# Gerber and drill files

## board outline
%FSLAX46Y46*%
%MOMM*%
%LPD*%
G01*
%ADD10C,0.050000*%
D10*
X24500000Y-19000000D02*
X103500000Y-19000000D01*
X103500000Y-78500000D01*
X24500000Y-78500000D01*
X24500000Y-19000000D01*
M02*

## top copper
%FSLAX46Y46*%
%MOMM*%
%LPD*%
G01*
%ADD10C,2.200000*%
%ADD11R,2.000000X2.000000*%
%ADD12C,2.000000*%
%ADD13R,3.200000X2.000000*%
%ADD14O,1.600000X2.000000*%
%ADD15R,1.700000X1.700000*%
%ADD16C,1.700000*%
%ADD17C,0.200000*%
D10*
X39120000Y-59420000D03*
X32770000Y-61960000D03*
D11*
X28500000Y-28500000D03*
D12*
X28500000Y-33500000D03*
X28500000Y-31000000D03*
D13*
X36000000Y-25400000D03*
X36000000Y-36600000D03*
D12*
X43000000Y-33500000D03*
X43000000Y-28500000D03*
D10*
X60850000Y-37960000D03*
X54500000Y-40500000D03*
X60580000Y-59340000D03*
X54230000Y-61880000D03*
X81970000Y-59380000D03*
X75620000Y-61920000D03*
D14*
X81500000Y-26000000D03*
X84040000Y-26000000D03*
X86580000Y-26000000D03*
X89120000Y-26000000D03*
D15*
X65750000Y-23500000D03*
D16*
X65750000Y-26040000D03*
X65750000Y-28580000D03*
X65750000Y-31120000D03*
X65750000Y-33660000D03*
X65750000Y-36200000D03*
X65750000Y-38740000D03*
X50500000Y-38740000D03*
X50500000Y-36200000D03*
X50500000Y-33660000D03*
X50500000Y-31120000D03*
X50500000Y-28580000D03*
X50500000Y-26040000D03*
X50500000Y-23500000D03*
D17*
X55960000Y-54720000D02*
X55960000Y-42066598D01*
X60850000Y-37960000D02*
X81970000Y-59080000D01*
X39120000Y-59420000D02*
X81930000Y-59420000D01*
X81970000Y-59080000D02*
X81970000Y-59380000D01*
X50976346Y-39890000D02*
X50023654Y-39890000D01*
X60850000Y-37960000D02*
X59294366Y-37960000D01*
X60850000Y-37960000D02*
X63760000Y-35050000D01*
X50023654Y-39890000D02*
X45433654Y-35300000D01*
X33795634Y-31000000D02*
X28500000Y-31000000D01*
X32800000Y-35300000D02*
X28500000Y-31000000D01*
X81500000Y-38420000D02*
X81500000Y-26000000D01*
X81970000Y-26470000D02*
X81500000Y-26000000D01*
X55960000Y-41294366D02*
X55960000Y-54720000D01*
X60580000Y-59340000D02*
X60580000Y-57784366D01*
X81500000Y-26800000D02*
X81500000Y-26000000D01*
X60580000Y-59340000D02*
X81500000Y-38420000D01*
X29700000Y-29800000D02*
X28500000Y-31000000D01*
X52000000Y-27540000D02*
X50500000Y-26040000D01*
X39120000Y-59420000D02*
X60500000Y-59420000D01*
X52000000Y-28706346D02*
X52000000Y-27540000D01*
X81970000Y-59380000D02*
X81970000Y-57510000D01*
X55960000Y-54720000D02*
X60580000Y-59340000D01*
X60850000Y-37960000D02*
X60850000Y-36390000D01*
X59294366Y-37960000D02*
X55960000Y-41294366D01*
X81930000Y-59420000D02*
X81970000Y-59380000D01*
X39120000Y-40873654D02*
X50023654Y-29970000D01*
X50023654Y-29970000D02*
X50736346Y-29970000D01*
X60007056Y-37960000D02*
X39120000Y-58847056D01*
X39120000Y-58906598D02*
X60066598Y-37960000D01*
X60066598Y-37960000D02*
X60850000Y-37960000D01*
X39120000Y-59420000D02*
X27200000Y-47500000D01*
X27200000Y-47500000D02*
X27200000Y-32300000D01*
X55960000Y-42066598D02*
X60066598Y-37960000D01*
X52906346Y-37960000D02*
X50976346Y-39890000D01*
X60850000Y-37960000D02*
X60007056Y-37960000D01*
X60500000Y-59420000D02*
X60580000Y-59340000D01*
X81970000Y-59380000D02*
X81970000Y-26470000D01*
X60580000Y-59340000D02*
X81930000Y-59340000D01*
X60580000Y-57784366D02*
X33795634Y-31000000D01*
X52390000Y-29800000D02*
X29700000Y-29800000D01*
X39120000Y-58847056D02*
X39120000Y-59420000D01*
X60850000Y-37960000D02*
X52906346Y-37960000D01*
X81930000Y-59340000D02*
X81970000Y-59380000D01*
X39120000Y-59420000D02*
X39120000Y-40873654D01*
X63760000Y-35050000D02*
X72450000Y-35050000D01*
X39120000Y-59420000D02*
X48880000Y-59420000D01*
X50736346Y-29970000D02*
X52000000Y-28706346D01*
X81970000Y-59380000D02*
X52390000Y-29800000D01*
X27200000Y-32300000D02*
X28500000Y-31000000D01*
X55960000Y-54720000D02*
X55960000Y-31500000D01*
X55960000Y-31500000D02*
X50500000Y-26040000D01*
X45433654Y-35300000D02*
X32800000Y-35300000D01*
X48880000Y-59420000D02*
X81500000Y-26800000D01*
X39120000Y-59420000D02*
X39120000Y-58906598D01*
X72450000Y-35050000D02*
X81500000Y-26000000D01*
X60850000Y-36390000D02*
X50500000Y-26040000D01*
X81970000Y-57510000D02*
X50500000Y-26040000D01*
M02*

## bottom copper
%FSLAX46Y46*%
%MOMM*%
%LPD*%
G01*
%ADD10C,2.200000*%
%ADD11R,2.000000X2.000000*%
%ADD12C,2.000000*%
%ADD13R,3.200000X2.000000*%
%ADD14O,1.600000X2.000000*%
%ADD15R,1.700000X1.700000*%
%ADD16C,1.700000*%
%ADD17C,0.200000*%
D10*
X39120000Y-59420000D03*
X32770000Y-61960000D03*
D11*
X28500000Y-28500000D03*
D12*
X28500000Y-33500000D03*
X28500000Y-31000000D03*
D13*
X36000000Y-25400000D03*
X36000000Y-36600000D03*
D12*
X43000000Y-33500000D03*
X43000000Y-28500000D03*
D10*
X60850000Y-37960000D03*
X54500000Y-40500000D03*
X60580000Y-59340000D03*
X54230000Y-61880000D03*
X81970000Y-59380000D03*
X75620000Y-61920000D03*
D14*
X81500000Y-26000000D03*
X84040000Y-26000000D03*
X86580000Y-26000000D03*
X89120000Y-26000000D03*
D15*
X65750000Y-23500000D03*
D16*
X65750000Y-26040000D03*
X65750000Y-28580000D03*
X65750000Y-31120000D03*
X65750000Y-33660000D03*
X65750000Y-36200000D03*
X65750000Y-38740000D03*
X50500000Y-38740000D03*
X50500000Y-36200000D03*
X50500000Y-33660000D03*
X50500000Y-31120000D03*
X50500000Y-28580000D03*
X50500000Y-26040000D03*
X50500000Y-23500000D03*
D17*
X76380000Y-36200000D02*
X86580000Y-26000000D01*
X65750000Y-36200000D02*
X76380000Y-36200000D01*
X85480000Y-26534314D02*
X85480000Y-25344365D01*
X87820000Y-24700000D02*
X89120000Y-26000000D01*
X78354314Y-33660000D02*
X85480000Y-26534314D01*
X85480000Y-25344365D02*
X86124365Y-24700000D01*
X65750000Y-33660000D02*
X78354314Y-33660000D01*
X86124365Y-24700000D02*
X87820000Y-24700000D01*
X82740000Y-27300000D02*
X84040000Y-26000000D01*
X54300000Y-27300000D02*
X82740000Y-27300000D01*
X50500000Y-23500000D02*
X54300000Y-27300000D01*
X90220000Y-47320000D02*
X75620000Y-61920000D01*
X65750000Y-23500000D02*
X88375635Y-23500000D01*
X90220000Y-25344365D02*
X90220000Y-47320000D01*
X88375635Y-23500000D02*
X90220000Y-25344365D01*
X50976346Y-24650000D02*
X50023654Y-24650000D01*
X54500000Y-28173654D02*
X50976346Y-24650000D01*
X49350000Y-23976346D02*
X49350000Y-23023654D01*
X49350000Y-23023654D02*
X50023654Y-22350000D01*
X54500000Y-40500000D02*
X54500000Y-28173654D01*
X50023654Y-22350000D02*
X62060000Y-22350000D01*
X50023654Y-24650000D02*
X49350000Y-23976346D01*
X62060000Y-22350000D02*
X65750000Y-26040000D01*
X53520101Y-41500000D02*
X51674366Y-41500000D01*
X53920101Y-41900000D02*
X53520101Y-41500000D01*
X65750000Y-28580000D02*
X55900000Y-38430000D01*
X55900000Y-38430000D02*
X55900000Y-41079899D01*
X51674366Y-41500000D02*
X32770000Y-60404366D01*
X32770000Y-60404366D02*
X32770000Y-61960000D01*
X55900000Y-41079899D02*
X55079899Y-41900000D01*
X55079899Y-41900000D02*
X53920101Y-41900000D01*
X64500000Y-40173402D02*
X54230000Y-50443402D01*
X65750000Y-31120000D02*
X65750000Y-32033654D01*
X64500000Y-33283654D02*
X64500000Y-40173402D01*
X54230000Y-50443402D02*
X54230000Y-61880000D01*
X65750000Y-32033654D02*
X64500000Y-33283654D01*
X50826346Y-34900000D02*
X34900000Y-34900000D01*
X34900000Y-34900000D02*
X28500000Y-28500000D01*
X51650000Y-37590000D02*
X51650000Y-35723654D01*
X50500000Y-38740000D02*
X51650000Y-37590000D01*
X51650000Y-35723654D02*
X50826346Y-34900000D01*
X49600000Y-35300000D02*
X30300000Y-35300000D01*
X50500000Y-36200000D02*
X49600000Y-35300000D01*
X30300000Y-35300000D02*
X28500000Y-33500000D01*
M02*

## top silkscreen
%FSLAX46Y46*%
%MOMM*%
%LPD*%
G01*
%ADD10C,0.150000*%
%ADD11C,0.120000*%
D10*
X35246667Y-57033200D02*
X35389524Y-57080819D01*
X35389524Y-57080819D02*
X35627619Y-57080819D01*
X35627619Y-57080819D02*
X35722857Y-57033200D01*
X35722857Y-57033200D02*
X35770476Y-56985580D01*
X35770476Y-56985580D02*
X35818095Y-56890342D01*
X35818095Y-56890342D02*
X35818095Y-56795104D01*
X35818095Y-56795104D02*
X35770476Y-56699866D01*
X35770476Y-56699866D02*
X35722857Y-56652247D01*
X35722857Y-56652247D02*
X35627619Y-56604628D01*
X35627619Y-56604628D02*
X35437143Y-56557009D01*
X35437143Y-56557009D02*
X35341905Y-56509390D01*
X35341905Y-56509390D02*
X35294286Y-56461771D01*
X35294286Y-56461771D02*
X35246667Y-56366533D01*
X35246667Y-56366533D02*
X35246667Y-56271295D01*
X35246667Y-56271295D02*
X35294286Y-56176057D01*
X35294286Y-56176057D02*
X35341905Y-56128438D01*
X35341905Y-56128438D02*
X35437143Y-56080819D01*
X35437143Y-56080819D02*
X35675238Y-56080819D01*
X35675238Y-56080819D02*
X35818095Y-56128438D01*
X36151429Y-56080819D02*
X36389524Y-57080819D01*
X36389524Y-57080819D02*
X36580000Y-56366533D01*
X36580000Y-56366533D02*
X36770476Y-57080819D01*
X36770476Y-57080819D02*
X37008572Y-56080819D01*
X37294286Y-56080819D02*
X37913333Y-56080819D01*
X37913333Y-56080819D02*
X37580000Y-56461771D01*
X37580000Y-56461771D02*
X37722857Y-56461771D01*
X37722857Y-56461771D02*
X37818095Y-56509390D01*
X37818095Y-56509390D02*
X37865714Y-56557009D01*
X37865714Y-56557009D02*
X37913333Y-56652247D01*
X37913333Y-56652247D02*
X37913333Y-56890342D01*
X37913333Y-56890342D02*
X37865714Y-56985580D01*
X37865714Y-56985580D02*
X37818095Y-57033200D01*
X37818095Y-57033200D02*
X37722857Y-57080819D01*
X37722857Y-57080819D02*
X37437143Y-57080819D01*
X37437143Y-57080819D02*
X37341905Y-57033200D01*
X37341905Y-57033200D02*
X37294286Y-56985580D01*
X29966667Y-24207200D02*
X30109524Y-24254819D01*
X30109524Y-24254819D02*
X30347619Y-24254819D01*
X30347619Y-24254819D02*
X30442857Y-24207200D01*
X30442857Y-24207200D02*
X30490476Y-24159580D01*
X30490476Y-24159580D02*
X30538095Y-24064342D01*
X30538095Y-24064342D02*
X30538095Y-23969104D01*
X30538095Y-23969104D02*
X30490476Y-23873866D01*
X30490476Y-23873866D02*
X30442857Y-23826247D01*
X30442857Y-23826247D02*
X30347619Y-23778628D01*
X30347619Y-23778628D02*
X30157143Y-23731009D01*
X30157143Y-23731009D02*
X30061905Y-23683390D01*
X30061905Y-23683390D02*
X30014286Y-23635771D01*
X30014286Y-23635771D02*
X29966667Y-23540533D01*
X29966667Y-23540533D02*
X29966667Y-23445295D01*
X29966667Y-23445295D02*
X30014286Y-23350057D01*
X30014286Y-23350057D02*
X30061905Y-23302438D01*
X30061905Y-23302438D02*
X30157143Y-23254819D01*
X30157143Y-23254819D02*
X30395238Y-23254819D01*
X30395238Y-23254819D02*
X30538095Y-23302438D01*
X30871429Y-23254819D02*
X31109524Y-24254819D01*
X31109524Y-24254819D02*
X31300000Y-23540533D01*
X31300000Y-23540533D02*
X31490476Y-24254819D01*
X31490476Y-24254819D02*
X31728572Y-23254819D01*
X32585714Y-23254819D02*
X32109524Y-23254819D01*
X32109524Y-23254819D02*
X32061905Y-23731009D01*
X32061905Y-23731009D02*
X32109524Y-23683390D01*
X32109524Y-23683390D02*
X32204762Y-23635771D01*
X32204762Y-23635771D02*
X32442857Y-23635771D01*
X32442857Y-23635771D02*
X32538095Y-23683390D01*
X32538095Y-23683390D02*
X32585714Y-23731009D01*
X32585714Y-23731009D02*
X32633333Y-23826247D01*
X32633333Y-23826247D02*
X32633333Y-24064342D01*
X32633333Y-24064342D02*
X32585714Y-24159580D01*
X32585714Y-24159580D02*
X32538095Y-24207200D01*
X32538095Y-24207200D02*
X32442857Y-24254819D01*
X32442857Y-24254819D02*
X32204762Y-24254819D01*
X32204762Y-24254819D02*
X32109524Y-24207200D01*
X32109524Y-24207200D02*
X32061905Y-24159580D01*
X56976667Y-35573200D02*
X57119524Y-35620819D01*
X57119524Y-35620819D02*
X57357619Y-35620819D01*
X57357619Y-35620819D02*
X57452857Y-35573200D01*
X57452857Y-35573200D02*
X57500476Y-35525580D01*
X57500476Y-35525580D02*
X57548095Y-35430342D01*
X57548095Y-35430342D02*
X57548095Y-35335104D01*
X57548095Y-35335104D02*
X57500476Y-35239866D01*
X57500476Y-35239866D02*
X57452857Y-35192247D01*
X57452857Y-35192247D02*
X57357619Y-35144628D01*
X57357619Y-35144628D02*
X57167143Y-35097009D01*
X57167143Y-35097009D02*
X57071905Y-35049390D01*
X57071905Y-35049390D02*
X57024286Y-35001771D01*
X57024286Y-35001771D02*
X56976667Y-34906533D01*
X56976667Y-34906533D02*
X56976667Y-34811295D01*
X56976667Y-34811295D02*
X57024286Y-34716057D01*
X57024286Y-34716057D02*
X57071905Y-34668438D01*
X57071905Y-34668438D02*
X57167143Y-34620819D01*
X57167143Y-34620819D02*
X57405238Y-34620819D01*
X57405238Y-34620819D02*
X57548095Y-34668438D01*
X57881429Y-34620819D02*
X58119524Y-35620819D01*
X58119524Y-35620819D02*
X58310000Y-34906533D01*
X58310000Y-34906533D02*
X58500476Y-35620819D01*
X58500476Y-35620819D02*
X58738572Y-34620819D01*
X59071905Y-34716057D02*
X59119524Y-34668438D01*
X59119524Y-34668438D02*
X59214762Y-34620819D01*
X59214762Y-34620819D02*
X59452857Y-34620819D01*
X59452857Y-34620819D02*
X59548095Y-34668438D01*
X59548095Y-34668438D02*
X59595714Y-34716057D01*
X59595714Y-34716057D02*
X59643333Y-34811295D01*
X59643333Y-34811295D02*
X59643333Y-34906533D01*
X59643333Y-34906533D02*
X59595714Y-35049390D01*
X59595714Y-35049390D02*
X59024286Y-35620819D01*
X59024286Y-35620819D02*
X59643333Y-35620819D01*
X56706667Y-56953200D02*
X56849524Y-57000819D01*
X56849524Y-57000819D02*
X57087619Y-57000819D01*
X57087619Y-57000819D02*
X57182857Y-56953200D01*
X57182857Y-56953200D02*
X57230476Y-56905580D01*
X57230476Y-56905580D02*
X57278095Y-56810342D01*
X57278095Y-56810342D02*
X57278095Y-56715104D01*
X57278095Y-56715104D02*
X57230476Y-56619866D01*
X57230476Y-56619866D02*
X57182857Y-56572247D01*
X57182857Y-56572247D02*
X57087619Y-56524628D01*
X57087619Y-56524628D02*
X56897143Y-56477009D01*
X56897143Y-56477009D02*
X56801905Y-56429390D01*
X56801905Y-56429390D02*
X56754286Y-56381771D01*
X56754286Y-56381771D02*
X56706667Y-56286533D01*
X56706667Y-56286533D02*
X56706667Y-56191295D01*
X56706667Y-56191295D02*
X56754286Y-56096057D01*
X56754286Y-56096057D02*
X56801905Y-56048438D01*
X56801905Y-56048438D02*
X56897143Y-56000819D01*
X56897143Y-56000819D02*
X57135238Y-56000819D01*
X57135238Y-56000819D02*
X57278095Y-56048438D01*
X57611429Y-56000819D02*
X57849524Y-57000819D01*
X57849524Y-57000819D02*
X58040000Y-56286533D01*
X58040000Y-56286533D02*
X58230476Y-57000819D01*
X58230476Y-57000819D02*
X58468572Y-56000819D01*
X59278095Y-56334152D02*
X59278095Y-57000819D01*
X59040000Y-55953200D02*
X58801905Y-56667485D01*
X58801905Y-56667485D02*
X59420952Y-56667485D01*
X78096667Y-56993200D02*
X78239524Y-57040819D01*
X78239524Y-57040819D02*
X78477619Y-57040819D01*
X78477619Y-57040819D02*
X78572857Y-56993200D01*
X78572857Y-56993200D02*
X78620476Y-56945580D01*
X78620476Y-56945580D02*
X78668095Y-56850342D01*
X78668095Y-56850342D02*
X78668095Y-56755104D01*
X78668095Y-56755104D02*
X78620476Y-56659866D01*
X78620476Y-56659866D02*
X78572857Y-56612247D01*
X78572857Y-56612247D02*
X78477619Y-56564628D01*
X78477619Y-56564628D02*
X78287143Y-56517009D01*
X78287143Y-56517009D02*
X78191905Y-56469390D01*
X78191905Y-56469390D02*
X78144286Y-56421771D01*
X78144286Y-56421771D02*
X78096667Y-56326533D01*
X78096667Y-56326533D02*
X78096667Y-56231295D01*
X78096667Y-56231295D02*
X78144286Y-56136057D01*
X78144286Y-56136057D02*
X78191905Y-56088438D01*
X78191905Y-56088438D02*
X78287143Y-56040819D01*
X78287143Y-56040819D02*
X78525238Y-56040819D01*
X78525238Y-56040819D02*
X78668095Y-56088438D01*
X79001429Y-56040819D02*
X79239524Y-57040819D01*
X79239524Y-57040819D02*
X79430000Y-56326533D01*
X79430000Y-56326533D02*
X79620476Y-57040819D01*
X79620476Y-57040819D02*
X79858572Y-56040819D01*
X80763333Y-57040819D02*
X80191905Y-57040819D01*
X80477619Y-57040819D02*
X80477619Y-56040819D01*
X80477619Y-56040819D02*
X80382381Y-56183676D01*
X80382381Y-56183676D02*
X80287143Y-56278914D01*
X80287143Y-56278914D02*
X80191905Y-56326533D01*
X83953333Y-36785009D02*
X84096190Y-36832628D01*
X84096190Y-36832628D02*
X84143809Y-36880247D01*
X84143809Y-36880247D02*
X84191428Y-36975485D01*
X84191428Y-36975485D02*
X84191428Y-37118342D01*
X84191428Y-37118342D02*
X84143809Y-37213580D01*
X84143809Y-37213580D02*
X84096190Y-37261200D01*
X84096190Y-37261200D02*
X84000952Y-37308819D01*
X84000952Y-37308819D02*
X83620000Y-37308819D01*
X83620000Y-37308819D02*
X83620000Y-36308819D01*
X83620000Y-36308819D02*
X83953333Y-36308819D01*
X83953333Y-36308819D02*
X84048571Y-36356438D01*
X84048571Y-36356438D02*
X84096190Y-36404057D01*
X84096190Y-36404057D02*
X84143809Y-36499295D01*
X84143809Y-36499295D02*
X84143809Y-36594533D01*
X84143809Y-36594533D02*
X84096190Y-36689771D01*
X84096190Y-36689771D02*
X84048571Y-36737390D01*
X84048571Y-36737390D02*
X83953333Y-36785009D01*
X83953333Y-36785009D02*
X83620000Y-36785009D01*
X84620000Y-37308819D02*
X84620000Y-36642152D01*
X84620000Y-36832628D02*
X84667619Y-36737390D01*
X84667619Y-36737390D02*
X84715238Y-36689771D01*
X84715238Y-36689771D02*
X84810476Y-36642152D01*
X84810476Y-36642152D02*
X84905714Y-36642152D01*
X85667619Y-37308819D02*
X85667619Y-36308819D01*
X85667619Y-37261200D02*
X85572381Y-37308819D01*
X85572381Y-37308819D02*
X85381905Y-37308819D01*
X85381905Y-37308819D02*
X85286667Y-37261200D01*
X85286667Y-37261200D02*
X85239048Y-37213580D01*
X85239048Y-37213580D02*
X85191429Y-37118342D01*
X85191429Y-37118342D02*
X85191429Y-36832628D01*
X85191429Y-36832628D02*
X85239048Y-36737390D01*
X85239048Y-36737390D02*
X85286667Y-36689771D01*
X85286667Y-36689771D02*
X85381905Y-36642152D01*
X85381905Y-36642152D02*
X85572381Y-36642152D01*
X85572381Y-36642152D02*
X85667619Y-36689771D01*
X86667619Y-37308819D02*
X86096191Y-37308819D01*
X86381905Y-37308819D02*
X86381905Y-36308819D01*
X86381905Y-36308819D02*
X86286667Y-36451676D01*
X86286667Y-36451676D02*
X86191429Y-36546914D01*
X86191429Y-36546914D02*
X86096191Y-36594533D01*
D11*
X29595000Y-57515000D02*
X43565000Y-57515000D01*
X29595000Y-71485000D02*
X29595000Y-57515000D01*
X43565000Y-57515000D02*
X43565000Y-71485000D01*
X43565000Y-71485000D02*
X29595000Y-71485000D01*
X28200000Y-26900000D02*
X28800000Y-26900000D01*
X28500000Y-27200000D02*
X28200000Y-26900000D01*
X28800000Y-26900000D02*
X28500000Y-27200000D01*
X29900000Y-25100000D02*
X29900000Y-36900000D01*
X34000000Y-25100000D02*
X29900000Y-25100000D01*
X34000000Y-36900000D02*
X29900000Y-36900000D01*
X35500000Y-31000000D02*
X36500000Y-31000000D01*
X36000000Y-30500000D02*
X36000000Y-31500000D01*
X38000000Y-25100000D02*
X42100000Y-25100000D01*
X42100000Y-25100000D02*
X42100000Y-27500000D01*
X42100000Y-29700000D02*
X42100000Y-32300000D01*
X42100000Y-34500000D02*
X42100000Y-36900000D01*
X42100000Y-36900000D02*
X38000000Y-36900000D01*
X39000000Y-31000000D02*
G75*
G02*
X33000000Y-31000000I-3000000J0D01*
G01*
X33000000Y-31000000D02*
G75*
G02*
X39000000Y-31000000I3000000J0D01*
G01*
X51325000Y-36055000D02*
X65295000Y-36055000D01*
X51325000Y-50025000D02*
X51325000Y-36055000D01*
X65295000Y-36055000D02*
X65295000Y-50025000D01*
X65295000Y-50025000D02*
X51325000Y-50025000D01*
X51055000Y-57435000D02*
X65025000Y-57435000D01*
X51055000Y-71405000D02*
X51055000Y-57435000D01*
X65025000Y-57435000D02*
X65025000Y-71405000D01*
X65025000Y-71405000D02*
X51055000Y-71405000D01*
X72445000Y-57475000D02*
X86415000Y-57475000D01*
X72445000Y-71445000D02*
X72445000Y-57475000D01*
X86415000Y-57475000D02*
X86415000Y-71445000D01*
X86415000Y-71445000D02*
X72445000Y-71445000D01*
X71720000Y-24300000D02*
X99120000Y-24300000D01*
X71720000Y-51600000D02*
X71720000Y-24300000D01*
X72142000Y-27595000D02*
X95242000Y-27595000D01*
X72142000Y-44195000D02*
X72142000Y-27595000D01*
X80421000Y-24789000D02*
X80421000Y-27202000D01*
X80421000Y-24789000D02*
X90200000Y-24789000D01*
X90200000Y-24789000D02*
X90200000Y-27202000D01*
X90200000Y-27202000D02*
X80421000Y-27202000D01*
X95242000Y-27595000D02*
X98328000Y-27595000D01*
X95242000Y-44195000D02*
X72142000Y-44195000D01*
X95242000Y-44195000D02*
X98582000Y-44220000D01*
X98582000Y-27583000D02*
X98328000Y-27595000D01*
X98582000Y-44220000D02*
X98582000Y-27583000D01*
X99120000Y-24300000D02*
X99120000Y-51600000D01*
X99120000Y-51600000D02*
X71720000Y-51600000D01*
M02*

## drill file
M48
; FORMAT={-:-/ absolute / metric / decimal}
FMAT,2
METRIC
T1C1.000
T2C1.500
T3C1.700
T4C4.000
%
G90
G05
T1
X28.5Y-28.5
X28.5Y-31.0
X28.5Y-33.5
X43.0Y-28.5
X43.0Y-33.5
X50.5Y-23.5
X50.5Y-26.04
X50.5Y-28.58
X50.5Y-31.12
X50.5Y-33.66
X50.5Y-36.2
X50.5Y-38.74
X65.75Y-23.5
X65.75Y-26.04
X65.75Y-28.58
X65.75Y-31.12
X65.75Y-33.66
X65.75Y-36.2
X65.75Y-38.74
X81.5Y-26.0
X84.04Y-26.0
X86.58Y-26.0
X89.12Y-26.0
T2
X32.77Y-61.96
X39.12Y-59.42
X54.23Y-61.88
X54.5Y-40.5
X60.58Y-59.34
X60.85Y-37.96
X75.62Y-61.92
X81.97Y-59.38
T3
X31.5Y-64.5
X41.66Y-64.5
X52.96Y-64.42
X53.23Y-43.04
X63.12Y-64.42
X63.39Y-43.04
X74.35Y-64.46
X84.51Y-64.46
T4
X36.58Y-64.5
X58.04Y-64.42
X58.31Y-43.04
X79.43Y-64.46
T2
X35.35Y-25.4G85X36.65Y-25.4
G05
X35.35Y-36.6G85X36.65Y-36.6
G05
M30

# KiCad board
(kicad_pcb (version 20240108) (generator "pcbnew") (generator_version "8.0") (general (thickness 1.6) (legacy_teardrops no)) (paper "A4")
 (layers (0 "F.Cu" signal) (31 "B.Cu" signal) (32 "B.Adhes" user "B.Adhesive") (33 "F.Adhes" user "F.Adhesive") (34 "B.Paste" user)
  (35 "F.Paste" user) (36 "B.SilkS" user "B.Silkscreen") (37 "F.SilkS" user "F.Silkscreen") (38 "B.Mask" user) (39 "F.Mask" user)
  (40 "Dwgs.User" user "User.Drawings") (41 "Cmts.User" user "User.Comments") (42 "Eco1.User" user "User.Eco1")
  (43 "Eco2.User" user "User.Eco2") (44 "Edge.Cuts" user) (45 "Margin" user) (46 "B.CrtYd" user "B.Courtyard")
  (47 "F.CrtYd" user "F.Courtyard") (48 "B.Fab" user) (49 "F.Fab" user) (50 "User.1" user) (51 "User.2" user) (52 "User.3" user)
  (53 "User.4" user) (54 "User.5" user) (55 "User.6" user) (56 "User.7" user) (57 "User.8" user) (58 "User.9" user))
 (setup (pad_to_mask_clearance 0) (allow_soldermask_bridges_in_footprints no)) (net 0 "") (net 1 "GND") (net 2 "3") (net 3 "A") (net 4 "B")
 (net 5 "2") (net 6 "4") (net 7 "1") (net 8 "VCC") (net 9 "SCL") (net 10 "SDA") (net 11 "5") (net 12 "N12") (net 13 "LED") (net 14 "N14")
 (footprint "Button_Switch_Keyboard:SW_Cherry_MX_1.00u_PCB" (layer "F.Cu") (at 39.12 59.42)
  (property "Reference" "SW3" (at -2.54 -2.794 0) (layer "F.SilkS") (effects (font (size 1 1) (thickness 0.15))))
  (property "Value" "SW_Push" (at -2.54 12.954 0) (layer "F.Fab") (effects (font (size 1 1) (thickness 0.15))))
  (fp_line (start -9.525 -1.905) (end 4.445 -1.905) (stroke (width 0.12) (type solid)) (layer "F.SilkS"))
  (fp_line (start -9.525 12.065) (end -9.525 -1.905) (stroke (width 0.12) (type solid)) (layer "F.SilkS"))
  (fp_line (start 4.445 -1.905) (end 4.445 12.065) (stroke (width 0.12) (type solid)) (layer "F.SilkS"))
  (fp_line (start 4.445 12.065) (end -9.525 12.065) (stroke (width 0.12) (type solid)) (layer "F.SilkS"))
  (pad "" np_thru_hole circle (at -7.62 5.08) (size 1.7 1.7) (drill 1.7) (layers "*.Cu" "*.Mask"))
  (pad "" np_thru_hole circle (at -2.54 5.08) (size 4 4) (drill 4) (layers "*.Cu" "*.Mask"))
  (pad "" np_thru_hole circle (at 2.54 5.08) (size 1.7 1.7) (drill 1.7) (layers "*.Cu" "*.Mask"))
  (pad "1" thru_hole circle (at 0 0) (size 2.2 2.2) (drill 1.5) (layers "*.Cu" "*.Mask") (remove_unused_layers no) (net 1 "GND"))
  (pad "2" thru_hole circle (at -6.35 2.54) (size 2.2 2.2) (drill 1.5) (layers "*.Cu" "*.Mask") (remove_unused_layers no) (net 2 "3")))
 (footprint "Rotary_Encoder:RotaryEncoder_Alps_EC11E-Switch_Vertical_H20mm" (layer "F.Cu") (at 28.5 28.5)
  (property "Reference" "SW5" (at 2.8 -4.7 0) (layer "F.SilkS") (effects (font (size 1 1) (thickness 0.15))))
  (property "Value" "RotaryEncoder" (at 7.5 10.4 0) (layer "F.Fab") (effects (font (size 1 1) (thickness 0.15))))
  (fp_line (start -0.3 -1.6) (end 0.3 -1.6) (stroke (width 0.12) (type solid)) (layer "F.SilkS"))
  (fp_line (start 0 -1.3) (end -0.3 -1.6) (stroke (width 0.12) (type solid)) (layer "F.SilkS"))
  (fp_line (start 0.3 -1.6) (end 0 -1.3) (stroke (width 0.12) (type solid)) (layer "F.SilkS"))
  (fp_line (start 1.4 -3.4) (end 1.4 8.4) (stroke (width 0.12) (type solid)) (layer "F.SilkS"))
  (fp_line (start 5.5 -3.4) (end 1.4 -3.4) (stroke (width 0.12) (type solid)) (layer "F.SilkS"))
  (fp_line (start 5.5 8.4) (end 1.4 8.4) (stroke (width 0.12) (type solid)) (layer "F.SilkS"))
  (fp_line (start 7 2.5) (end 8 2.5) (stroke (width 0.12) (type solid)) (layer "F.SilkS"))
  (fp_line (start 7.5 2) (end 7.5 3) (stroke (width 0.12) (type solid)) (layer "F.SilkS"))
  (fp_line (start 9.5 -3.4) (end 13.6 -3.4) (stroke (width 0.12) (type solid)) (layer "F.SilkS"))
  (fp_line (start 13.6 -3.4) (end 13.6 -1) (stroke (width 0.12) (type solid)) (layer "F.SilkS"))
  (fp_line (start 13.6 1.2) (end 13.6 3.8) (stroke (width 0.12) (type solid)) (layer "F.SilkS"))
  (fp_line (start 13.6 6) (end 13.6 8.4) (stroke (width 0.12) (type solid)) (layer "F.SilkS"))
  (fp_line (start 13.6 8.4) (end 9.5 8.4) (stroke (width 0.12) (type solid)) (layer "F.SilkS"))
  (fp_circle (center 7.5 2.5) (end 10.5 2.5) (stroke (width 0.12) (type solid)) (fill none) (layer "F.SilkS"))
  (pad "A" thru_hole rect (at 0 0) (size 2 2) (drill 1) (layers "*.Cu" "*.Mask") (remove_unused_layers no) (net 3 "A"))
  (pad "B" thru_hole circle (at 0 5) (size 2 2) (drill 1) (layers "*.Cu" "*.Mask") (remove_unused_layers no) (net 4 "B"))
  (pad "C" thru_hole circle (at 0 2.5) (size 2 2) (drill 1) (layers "*.Cu" "*.Mask") (remove_unused_layers no) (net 1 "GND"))
  (pad "MP" thru_hole rect (at 7.5 -3.1) (size 3.2 2) (drill oval 2.8 1.5) (layers "*.Cu" "*.Mask") (remove_unused_layers no))
  (pad "MP" thru_hole rect (at 7.5 8.1) (size 3.2 2) (drill oval 2.8 1.5) (layers "*.Cu" "*.Mask") (remove_unused_layers no))
  (pad "S1" thru_hole circle (at 14.5 5) (size 2 2) (drill 1) (layers "*.Cu" "*.Mask") (remove_unused_layers no))
  (pad "S2" thru_hole circle (at 14.5 0) (size 2 2) (drill 1) (layers "*.Cu" "*.Mask") (remove_unused_layers no)))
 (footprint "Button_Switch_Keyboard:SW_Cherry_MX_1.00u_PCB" (layer "F.Cu") (at 60.85 37.96)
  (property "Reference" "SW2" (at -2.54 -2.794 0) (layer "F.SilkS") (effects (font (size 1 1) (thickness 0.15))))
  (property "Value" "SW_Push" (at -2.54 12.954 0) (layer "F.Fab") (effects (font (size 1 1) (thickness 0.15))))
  (fp_line (start -9.525 -1.905) (end 4.445 -1.905) (stroke (width 0.12) (type solid)) (layer "F.SilkS"))
  (fp_line (start -9.525 12.065) (end -9.525 -1.905) (stroke (width 0.12) (type solid)) (layer "F.SilkS"))
  (fp_line (start 4.445 -1.905) (end 4.445 12.065) (stroke (width 0.12) (type solid)) (layer "F.SilkS"))
  (fp_line (start 4.445 12.065) (end -9.525 12.065) (stroke (width 0.12) (type solid)) (layer "F.SilkS"))
  (pad "" np_thru_hole circle (at -7.62 5.08) (size 1.7 1.7) (drill 1.7) (layers "*.Cu" "*.Mask"))
  (pad "" np_thru_hole circle (at -2.54 5.08) (size 4 4) (drill 4) (layers "*.Cu" "*.Mask"))
  (pad "" np_thru_hole circle (at 2.54 5.08) (size 1.7 1.7) (drill 1.7) (layers "*.Cu" "*.Mask"))
  (pad "1" thru_hole circle (at 0 0) (size 2.2 2.2) (drill 1.5) (layers "*.Cu" "*.Mask") (remove_unused_layers no) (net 1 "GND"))
  (pad "2" thru_hole circle (at -6.35 2.54) (size 2.2 2.2) (drill 1.5) (layers "*.Cu" "*.Mask") (remove_unused_layers no) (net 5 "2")))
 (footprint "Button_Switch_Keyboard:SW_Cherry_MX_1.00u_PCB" (layer "F.Cu") (at 60.58 59.34)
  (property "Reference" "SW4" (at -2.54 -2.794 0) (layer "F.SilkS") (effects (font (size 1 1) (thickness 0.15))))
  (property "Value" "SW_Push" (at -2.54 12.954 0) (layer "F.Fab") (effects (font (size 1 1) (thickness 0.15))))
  (fp_line (start -9.525 -1.905) (end 4.445 -1.905) (stroke (width 0.12) (type solid)) (layer "F.SilkS"))
  (fp_line (start -9.525 12.065) (end -9.525 -1.905) (stroke (width 0.12) (type solid)) (layer "F.SilkS"))
  (fp_line (start 4.445 -1.905) (end 4.445 12.065) (stroke (width 0.12) (type solid)) (layer "F.SilkS"))
  (fp_line (start 4.445 12.065) (end -9.525 12.065) (stroke (width 0.12) (type solid)) (layer "F.SilkS"))
  (pad "" np_thru_hole circle (at -7.62 5.08) (size 1.7 1.7) (drill 1.7) (layers "*.Cu" "*.Mask"))
  (pad "" np_thru_hole circle (at -2.54 5.08) (size 4 4) (drill 4) (layers "*.Cu" "*.Mask"))
  (pad "" np_thru_hole circle (at 2.54 5.08) (size 1.7 1.7) (drill 1.7) (layers "*.Cu" "*.Mask"))
  (pad "1" thru_hole circle (at 0 0) (size 2.2 2.2) (drill 1.5) (layers "*.Cu" "*.Mask") (remove_unused_layers no) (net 1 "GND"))
  (pad "2" thru_hole circle (at -6.35 2.54) (size 2.2 2.2) (drill 1.5) (layers "*.Cu" "*.Mask") (remove_unused_layers no) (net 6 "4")))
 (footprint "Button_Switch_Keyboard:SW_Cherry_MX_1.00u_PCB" (layer "F.Cu") (at 81.97 59.38)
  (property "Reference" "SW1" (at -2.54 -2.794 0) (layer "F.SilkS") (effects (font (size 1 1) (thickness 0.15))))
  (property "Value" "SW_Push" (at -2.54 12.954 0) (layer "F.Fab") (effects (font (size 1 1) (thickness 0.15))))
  (fp_line (start -9.525 -1.905) (end 4.445 -1.905) (stroke (width 0.12) (type solid)) (layer "F.SilkS"))
  (fp_line (start -9.525 12.065) (end -9.525 -1.905) (stroke (width 0.12) (type solid)) (layer "F.SilkS"))
  (fp_line (start 4.445 -1.905) (end 4.445 12.065) (stroke (width 0.12) (type solid)) (layer "F.SilkS"))
  (fp_line (start 4.445 12.065) (end -9.525 12.065) (stroke (width 0.12) (type solid)) (layer "F.SilkS"))
  (pad "" np_thru_hole circle (at -7.62 5.08) (size 1.7 1.7) (drill 1.7) (layers "*.Cu" "*.Mask"))
  (pad "" np_thru_hole circle (at -2.54 5.08) (size 4 4) (drill 4) (layers "*.Cu" "*.Mask"))
  (pad "" np_thru_hole circle (at 2.54 5.08) (size 1.7 1.7) (drill 1.7) (layers "*.Cu" "*.Mask"))
  (pad "1" thru_hole circle (at 0 0) (size 2.2 2.2) (drill 1.5) (layers "*.Cu" "*.Mask") (remove_unused_layers no) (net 1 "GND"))
  (pad "2" thru_hole circle (at -6.35 2.54) (size 2.2 2.2) (drill 1.5) (layers "*.Cu" "*.Mask") (remove_unused_layers no) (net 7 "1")))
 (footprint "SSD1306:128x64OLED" (layer "F.Cu") (at 85.12 36.6)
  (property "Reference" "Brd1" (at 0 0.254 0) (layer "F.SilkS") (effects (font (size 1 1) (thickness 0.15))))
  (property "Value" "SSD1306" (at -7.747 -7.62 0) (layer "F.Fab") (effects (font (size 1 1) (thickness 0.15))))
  (fp_line (start -13.4 -12.3) (end 14 -12.3) (stroke (width 0.12) (type solid)) (layer "F.SilkS"))
  (fp_line (start -13.4 15) (end -13.4 -12.3) (stroke (width 0.12) (type solid)) (layer "F.SilkS"))
  (fp_line (start -12.978 -9.005) (end 10.122 -9.005) (stroke (width 0.12) (type solid)) (layer "F.SilkS"))
  (fp_line (start -12.978 7.595) (end -12.978 -9.005) (stroke (width 0.12) (type solid)) (layer "F.SilkS"))
  (fp_line (start -4.699 -11.811) (end -4.699 -9.398) (stroke (width 0.12) (type solid)) (layer "F.SilkS"))
  (fp_line (start -4.699 -11.811) (end 5.08 -11.811) (stroke (width 0.12) (type solid)) (layer "F.SilkS"))
  (fp_line (start 5.08 -11.811) (end 5.08 -9.398) (stroke (width 0.12) (type solid)) (layer "F.SilkS"))
  (fp_line (start 5.08 -9.398) (end -4.699 -9.398) (stroke (width 0.12) (type solid)) (layer "F.SilkS"))
  (fp_line (start 10.122 -9.005) (end 13.208 -9.005) (stroke (width 0.12) (type solid)) (layer "F.SilkS"))
  (fp_line (start 10.122 7.595) (end -12.978 7.595) (stroke (width 0.12) (type solid)) (layer "F.SilkS"))
  (fp_line (start 10.122 7.595) (end 13.462 7.62) (stroke (width 0.12) (type solid)) (layer "F.SilkS"))
  (fp_line (start 13.462 -9.017) (end 13.208 -9.005) (stroke (width 0.12) (type solid)) (layer "F.SilkS"))
  (fp_line (start 13.462 7.62) (end 13.462 -9.017) (stroke (width 0.12) (type solid)) (layer "F.SilkS"))
  (fp_line (start 14 -12.3) (end 14 15) (stroke (width 0.12) (type solid)) (layer "F.SilkS"))
  (fp_line (start 14 15) (end -13.4 15) (stroke (width 0.12) (type solid)) (layer "F.SilkS"))
  (pad "1" thru_hole oval (at -3.62 -10.6 90) (size 2 1.6) (drill 1) (layers "*.Cu" "*.Mask") (remove_unused_layers no) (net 1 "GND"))
  (pad "2" thru_hole oval (at -1.08 -10.6 90) (size 2 1.6) (drill 1) (layers "*.Cu" "*.Mask") (remove_unused_layers no) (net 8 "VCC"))
  (pad "3" thru_hole oval (at 1.46 -10.6 90) (size 2 1.6) (drill 1) (layers "*.Cu" "*.Mask") (remove_unused_layers no) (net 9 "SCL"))
  (pad "4" thru_hole oval (at 4 -10.6 90) (size 2 1.6) (drill 1) (layers "*.Cu" "*.Mask") (remove_unused_layers no) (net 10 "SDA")))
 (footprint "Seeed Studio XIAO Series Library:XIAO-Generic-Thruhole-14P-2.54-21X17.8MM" (layer "B.Cu") (at 58.125 31.12 180)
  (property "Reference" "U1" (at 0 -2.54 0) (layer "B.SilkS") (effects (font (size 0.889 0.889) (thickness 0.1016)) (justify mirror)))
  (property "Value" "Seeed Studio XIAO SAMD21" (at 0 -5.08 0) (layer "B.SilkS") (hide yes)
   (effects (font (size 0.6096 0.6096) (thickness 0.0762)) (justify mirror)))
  (pad "1" thru_hole rect (at -7.625 7.62 180) (size 1.7 1.7) (drill 1) (layers "*.Cu" "*.Mask") (remove_unused_layers no) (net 7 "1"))
  (pad "2" thru_hole circle (at -7.625 5.08 180) (size 1.7 1.7) (drill 1) (layers "*.Cu" "*.Mask") (remove_unused_layers no) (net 5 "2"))
  (pad "3" thru_hole circle (at -7.625 2.54 180) (size 1.7 1.7) (drill 1) (layers "*.Cu" "*.Mask") (remove_unused_layers no) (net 2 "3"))
  (pad "4" thru_hole circle (at -7.625 0 180) (size 1.7 1.7) (drill 1) (layers "*.Cu" "*.Mask") (remove_unused_layers no) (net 6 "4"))
  (pad "5" thru_hole circle (at -7.625 -2.54 180) (size 1.7 1.7) (drill 1) (layers "*.Cu" "*.Mask") (remove_unused_layers no) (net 10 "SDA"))
  (pad "6" thru_hole circle (at -7.625 -5.08) (size 1.7 1.7) (drill 1) (layers "*.Cu" "*.Mask") (remove_unused_layers no) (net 9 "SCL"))
  (pad "7" thru_hole circle (at -7.625 -7.62 180) (size 1.7 1.7) (drill 1) (layers "*.Cu" "*.Mask") (remove_unused_layers no) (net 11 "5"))
  (pad "8" thru_hole circle (at 7.625 -7.62 180) (size 1.7 1.7) (drill 1) (layers "*.Cu" "*.Mask") (remove_unused_layers no) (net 3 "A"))
  (pad "9" thru_hole circle (at 7.625 -5.08 180) (size 1.7 1.7) (drill 1) (layers "*.Cu" "*.Mask") (remove_unused_layers no) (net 4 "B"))
  (pad "10" thru_hole circle (at 7.625 -2.54 180) (size 1.7 1.7) (drill 1) (layers "*.Cu" "*.Mask") (remove_unused_layers no) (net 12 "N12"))
  (pad "11" thru_hole circle (at 7.625 0 180) (size 1.7 1.7) (drill 1) (layers "*.Cu" "*.Mask") (remove_unused_layers no) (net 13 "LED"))
  (pad "12" thru_hole circle (at 7.625 2.54 180) (size 1.7 1.7) (drill 1) (layers "*.Cu" "*.Mask") (remove_unused_layers no) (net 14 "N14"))
  (pad "13" thru_hole circle (at 7.625 5.08 180) (size 1.7 1.7) (drill 1) (layers "*.Cu" "*.Mask") (remove_unused_layers no) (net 1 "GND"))
  (pad "14" thru_hole circle (at 7.625 7.62 180) (size 1.7 1.7) (drill 1) (layers "*.Cu" "*.Mask") (remove_unused_layers no) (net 8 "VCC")))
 (gr_rect (start 24.5 19) (end 103.5 78.5) (stroke (width 0.05) (type default)) (fill none) (layer "Edge.Cuts"))
 (segment (start 76.38 36.2) (end 86.58 26) (width 0.2) (layer "B.Cu") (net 9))
 (segment (start 65.75 36.2) (end 76.38 36.2) (width 0.2) (layer "B.Cu") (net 9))
 (segment (start 85.48 26.534314) (end 85.48 25.344365) (width 0.2) (layer "B.Cu") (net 10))
 (segment (start 87.82 24.7) (end 89.12 26) (width 0.2) (layer "B.Cu") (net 10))
 (segment (start 78.354314 33.66) (end 85.48 26.534314) (width 0.2) (layer "B.Cu") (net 10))
 (segment (start 85.48 25.344365) (end 86.124365 24.7) (width 0.2) (layer "B.Cu") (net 10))
 (segment (start 65.75 33.66) (end 78.354314 33.66) (width 0.2) (layer "B.Cu") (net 10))
 (segment (start 86.124365 24.7) (end 87.82 24.7) (width 0.2) (layer "B.Cu") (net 10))
 (segment (start 55.96 54.72) (end 55.96 42.066598) (width 0.2) (layer "F.Cu") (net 1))
 (segment (start 60.85 37.96) (end 81.97 59.08) (width 0.2) (layer "F.Cu") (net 1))
 (segment (start 39.12 59.42) (end 81.93 59.42) (width 0.2) (layer "F.Cu") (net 1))
 (segment (start 81.97 59.08) (end 81.97 59.38) (width 0.2) (layer "F.Cu") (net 1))
 (segment (start 50.976346 39.89) (end 50.023654 39.89) (width 0.2) (layer "F.Cu") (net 1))
 (segment (start 60.85 37.96) (end 59.294366 37.96) (width 0.2) (layer "F.Cu") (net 1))
 (segment (start 60.85 37.96) (end 63.76 35.05) (width 0.2) (layer "F.Cu") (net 1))
 (segment (start 50.023654 39.89) (end 45.433654 35.3) (width 0.2) (layer "F.Cu") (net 1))
 (segment (start 33.795634 31) (end 28.5 31) (width 0.2) (layer "F.Cu") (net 1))
 (segment (start 32.8 35.3) (end 28.5 31) (width 0.2) (layer "F.Cu") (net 1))
 (segment (start 81.5 38.42) (end 81.5 26) (width 0.2) (layer "F.Cu") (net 1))
 (segment (start 81.97 26.47) (end 81.5 26) (width 0.2) (layer "F.Cu") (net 1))
 (segment (start 55.96 41.294366) (end 55.96 54.72) (width 0.2) (layer "F.Cu") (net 1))
 (segment (start 60.58 59.34) (end 60.58 57.784366) (width 0.2) (layer "F.Cu") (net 1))
 (segment (start 81.5 26.8) (end 81.5 26) (width 0.2) (layer "F.Cu") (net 1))
 (segment (start 60.58 59.34) (end 81.5 38.42) (width 0.2) (layer "F.Cu") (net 1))
 (segment (start 29.7 29.8) (end 28.5 31) (width 0.2) (layer "F.Cu") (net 1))
 (segment (start 52 27.54) (end 50.5 26.04) (width 0.2) (layer "F.Cu") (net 1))
 (segment (start 39.12 59.42) (end 60.5 59.42) (width 0.2) (layer "F.Cu") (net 1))
 (segment (start 52 28.706346) (end 52 27.54) (width 0.2) (layer "F.Cu") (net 1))
 (segment (start 81.97 59.38) (end 81.97 57.51) (width 0.2) (layer "F.Cu") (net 1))
 (segment (start 55.96 54.72) (end 60.58 59.34) (width 0.2) (layer "F.Cu") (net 1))
 (segment (start 60.85 37.96) (end 60.85 36.39) (width 0.2) (layer "F.Cu") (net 1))
 (segment (start 59.294366 37.96) (end 55.96 41.294366) (width 0.2) (layer "F.Cu") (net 1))
 (segment (start 81.93 59.42) (end 81.97 59.38) (width 0.2) (layer "F.Cu") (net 1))
 (segment (start 39.12 40.873654) (end 50.023654 29.97) (width 0.2) (layer "F.Cu") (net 1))
 (segment (start 50.023654 29.97) (end 50.736346 29.97) (width 0.2) (layer "F.Cu") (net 1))
 (segment (start 60.007056 37.96) (end 39.12 58.847056) (width 0.2) (layer "F.Cu") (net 1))
 (segment (start 39.12 58.906598) (end 60.066598 37.96) (width 0.2) (layer "F.Cu") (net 1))
 (segment (start 60.066598 37.96) (end 60.85 37.96) (width 0.2) (layer "F.Cu") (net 1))
 (segment (start 39.12 59.42) (end 27.2 47.5) (width 0.2) (layer "F.Cu") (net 1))
 (segment (start 27.2 47.5) (end 27.2 32.3) (width 0.2) (layer "F.Cu") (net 1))
 (segment (start 55.96 42.066598) (end 60.066598 37.96) (width 0.2) (layer "F.Cu") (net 1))
 (segment (start 52.906346 37.96) (end 50.976346 39.89) (width 0.2) (layer "F.Cu") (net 1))
 (segment (start 60.85 37.96) (end 60.007056 37.96) (width 0.2) (layer "F.Cu") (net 1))
 (segment (start 60.5 59.42) (end 60.58 59.34) (width 0.2) (layer "F.Cu") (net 1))
 (segment (start 81.97 59.38) (end 81.97 26.47) (width 0.2) (layer "F.Cu") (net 1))
 (segment (start 60.58 59.34) (end 81.93 59.34) (width 0.2) (layer "F.Cu") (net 1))
 (segment (start 60.58 57.784366) (end 33.795634 31) (width 0.2) (layer "F.Cu") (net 1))
 (segment (start 52.39 29.8) (end 29.7 29.8) (width 0.2) (layer "F.Cu") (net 1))
 (segment (start 39.12 58.847056) (end 39.12 59.42) (width 0.2) (layer "F.Cu") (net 1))
 (segment (start 60.85 37.96) (end 52.906346 37.96) (width 0.2) (layer "F.Cu") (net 1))
 (segment (start 81.93 59.34) (end 81.97 59.38) (width 0.2) (layer "F.Cu") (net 1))
 (segment (start 39.12 59.42) (end 39.12 40.873654) (width 0.2) (layer "F.Cu") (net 1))
 (segment (start 63.76 35.05) (end 72.45 35.05) (width 0.2) (layer "F.Cu") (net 1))
 (segment (start 39.12 59.42) (end 48.88 59.42) (width 0.2) (layer "F.Cu") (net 1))
 (segment (start 50.736346 29.97) (end 52 28.706346) (width 0.2) (layer "F.Cu") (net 1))
 (segment (start 81.97 59.38) (end 52.39 29.8) (width 0.2) (layer "F.Cu") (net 1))
 (segment (start 27.2 32.3) (end 28.5 31) (width 0.2) (layer "F.Cu") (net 1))
 (segment (start 55.96 54.72) (end 55.96 31.5) (width 0.2) (layer "F.Cu") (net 1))
 (segment (start 55.96 31.5) (end 50.5 26.04) (width 0.2) (layer "F.Cu") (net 1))
 (segment (start 45.433654 35.3) (end 32.8 35.3) (width 0.2) (layer "F.Cu") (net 1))
 (segment (start 48.88 59.42) (end 81.5 26.8) (width 0.2) (layer "F.Cu") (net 1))
 (segment (start 39.12 59.42) (end 39.12 58.906598) (width 0.2) (layer "F.Cu") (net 1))
 (segment (start 72.45 35.05) (end 81.5 26) (width 0.2) (layer "F.Cu") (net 1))
 (segment (start 60.85 36.39) (end 50.5 26.04) (width 0.2) (layer "F.Cu") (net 1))
 (segment (start 81.97 57.51) (end 50.5 26.04) (width 0.2) (layer "F.Cu") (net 1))
 (segment (start 82.74 27.3) (end 84.04 26) (width 0.2) (layer "B.Cu") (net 8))
 (segment (start 54.3 27.3) (end 82.74 27.3) (width 0.2) (layer "B.Cu") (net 8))
 (segment (start 50.5 23.5) (end 54.3 27.3) (width 0.2) (layer "B.Cu") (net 8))
 (segment (start 90.22 47.32) (end 75.62 61.92) (width 0.2) (layer "B.Cu") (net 7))
 (segment (start 65.75 23.5) (end 88.375635 23.5) (width 0.2) (layer "B.Cu") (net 7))
 (segment (start 90.22 25.344365) (end 90.22 47.32) (width 0.2) (layer "B.Cu") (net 7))
 (segment (start 88.375635 23.5) (end 90.22 25.344365) (width 0.2) (layer "B.Cu") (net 7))
 (segment (start 50.976346 24.65) (end 50.023654 24.65) (width 0.2) (layer "B.Cu") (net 5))
 (segment (start 54.5 28.173654) (end 50.976346 24.65) (width 0.2) (layer "B.Cu") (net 5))
 (segment (start 49.35 23.976346) (end 49.35 23.023654) (width 0.2) (layer "B.Cu") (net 5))
 (segment (start 49.35 23.023654) (end 50.023654 22.35) (width 0.2) (layer "B.Cu") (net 5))
 (segment (start 54.5 40.5) (end 54.5 28.173654) (width 0.2) (layer "B.Cu") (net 5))
 (segment (start 50.023654 22.35) (end 62.06 22.35) (width 0.2) (layer "B.Cu") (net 5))
 (segment (start 50.023654 24.65) (end 49.35 23.976346) (width 0.2) (layer "B.Cu") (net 5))
 (segment (start 62.06 22.35) (end 65.75 26.04) (width 0.2) (layer "B.Cu") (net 5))
 (segment (start 53.520101 41.5) (end 51.674366 41.5) (width 0.2) (layer "B.Cu") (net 2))
 (segment (start 53.920101 41.9) (end 53.520101 41.5) (width 0.2) (layer "B.Cu") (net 2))
 (segment (start 65.75 28.58) (end 55.9 38.43) (width 0.2) (layer "B.Cu") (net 2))
 (segment (start 55.9 38.43) (end 55.9 41.079899) (width 0.2) (layer "B.Cu") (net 2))
 (segment (start 51.674366 41.5) (end 32.77 60.404366) (width 0.2) (layer "B.Cu") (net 2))
 (segment (start 32.77 60.404366) (end 32.77 61.96) (width 0.2) (layer "B.Cu") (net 2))
 (segment (start 55.9 41.079899) (end 55.079899 41.9) (width 0.2) (layer "B.Cu") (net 2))
 (segment (start 55.079899 41.9) (end 53.920101 41.9) (width 0.2) (layer "B.Cu") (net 2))
 (segment (start 64.5 40.173402) (end 54.23 50.443402) (width 0.2) (layer "B.Cu") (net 6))
 (segment (start 65.75 31.12) (end 65.75 32.033654) (width 0.2) (layer "B.Cu") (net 6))
 (segment (start 64.5 33.283654) (end 64.5 40.173402) (width 0.2) (layer "B.Cu") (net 6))
 (segment (start 54.23 50.443402) (end 54.23 61.88) (width 0.2) (layer "B.Cu") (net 6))
 (segment (start 65.75 32.033654) (end 64.5 33.283654) (width 0.2) (layer "B.Cu") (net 6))
 (segment (start 50.826346 34.9) (end 34.9 34.9) (width 0.2) (layer "B.Cu") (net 3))
 (segment (start 34.9 34.9) (end 28.5 28.5) (width 0.2) (layer "B.Cu") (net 3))
 (segment (start 51.65 37.59) (end 51.65 35.723654) (width 0.2) (layer "B.Cu") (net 3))
 (segment (start 50.5 38.74) (end 51.65 37.59) (width 0.2) (layer "B.Cu") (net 3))
 (segment (start 51.65 35.723654) (end 50.826346 34.9) (width 0.2) (layer "B.Cu") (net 3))
 (segment (start 49.6 35.3) (end 30.3 35.3) (width 0.2) (layer "B.Cu") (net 4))
 (segment (start 50.5 36.2) (end 49.6 35.3) (width 0.2) (layer "B.Cu") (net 4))
 (segment (start 30.3 35.3) (end 28.5 33.5) (width 0.2) (layer "B.Cu") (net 4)))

